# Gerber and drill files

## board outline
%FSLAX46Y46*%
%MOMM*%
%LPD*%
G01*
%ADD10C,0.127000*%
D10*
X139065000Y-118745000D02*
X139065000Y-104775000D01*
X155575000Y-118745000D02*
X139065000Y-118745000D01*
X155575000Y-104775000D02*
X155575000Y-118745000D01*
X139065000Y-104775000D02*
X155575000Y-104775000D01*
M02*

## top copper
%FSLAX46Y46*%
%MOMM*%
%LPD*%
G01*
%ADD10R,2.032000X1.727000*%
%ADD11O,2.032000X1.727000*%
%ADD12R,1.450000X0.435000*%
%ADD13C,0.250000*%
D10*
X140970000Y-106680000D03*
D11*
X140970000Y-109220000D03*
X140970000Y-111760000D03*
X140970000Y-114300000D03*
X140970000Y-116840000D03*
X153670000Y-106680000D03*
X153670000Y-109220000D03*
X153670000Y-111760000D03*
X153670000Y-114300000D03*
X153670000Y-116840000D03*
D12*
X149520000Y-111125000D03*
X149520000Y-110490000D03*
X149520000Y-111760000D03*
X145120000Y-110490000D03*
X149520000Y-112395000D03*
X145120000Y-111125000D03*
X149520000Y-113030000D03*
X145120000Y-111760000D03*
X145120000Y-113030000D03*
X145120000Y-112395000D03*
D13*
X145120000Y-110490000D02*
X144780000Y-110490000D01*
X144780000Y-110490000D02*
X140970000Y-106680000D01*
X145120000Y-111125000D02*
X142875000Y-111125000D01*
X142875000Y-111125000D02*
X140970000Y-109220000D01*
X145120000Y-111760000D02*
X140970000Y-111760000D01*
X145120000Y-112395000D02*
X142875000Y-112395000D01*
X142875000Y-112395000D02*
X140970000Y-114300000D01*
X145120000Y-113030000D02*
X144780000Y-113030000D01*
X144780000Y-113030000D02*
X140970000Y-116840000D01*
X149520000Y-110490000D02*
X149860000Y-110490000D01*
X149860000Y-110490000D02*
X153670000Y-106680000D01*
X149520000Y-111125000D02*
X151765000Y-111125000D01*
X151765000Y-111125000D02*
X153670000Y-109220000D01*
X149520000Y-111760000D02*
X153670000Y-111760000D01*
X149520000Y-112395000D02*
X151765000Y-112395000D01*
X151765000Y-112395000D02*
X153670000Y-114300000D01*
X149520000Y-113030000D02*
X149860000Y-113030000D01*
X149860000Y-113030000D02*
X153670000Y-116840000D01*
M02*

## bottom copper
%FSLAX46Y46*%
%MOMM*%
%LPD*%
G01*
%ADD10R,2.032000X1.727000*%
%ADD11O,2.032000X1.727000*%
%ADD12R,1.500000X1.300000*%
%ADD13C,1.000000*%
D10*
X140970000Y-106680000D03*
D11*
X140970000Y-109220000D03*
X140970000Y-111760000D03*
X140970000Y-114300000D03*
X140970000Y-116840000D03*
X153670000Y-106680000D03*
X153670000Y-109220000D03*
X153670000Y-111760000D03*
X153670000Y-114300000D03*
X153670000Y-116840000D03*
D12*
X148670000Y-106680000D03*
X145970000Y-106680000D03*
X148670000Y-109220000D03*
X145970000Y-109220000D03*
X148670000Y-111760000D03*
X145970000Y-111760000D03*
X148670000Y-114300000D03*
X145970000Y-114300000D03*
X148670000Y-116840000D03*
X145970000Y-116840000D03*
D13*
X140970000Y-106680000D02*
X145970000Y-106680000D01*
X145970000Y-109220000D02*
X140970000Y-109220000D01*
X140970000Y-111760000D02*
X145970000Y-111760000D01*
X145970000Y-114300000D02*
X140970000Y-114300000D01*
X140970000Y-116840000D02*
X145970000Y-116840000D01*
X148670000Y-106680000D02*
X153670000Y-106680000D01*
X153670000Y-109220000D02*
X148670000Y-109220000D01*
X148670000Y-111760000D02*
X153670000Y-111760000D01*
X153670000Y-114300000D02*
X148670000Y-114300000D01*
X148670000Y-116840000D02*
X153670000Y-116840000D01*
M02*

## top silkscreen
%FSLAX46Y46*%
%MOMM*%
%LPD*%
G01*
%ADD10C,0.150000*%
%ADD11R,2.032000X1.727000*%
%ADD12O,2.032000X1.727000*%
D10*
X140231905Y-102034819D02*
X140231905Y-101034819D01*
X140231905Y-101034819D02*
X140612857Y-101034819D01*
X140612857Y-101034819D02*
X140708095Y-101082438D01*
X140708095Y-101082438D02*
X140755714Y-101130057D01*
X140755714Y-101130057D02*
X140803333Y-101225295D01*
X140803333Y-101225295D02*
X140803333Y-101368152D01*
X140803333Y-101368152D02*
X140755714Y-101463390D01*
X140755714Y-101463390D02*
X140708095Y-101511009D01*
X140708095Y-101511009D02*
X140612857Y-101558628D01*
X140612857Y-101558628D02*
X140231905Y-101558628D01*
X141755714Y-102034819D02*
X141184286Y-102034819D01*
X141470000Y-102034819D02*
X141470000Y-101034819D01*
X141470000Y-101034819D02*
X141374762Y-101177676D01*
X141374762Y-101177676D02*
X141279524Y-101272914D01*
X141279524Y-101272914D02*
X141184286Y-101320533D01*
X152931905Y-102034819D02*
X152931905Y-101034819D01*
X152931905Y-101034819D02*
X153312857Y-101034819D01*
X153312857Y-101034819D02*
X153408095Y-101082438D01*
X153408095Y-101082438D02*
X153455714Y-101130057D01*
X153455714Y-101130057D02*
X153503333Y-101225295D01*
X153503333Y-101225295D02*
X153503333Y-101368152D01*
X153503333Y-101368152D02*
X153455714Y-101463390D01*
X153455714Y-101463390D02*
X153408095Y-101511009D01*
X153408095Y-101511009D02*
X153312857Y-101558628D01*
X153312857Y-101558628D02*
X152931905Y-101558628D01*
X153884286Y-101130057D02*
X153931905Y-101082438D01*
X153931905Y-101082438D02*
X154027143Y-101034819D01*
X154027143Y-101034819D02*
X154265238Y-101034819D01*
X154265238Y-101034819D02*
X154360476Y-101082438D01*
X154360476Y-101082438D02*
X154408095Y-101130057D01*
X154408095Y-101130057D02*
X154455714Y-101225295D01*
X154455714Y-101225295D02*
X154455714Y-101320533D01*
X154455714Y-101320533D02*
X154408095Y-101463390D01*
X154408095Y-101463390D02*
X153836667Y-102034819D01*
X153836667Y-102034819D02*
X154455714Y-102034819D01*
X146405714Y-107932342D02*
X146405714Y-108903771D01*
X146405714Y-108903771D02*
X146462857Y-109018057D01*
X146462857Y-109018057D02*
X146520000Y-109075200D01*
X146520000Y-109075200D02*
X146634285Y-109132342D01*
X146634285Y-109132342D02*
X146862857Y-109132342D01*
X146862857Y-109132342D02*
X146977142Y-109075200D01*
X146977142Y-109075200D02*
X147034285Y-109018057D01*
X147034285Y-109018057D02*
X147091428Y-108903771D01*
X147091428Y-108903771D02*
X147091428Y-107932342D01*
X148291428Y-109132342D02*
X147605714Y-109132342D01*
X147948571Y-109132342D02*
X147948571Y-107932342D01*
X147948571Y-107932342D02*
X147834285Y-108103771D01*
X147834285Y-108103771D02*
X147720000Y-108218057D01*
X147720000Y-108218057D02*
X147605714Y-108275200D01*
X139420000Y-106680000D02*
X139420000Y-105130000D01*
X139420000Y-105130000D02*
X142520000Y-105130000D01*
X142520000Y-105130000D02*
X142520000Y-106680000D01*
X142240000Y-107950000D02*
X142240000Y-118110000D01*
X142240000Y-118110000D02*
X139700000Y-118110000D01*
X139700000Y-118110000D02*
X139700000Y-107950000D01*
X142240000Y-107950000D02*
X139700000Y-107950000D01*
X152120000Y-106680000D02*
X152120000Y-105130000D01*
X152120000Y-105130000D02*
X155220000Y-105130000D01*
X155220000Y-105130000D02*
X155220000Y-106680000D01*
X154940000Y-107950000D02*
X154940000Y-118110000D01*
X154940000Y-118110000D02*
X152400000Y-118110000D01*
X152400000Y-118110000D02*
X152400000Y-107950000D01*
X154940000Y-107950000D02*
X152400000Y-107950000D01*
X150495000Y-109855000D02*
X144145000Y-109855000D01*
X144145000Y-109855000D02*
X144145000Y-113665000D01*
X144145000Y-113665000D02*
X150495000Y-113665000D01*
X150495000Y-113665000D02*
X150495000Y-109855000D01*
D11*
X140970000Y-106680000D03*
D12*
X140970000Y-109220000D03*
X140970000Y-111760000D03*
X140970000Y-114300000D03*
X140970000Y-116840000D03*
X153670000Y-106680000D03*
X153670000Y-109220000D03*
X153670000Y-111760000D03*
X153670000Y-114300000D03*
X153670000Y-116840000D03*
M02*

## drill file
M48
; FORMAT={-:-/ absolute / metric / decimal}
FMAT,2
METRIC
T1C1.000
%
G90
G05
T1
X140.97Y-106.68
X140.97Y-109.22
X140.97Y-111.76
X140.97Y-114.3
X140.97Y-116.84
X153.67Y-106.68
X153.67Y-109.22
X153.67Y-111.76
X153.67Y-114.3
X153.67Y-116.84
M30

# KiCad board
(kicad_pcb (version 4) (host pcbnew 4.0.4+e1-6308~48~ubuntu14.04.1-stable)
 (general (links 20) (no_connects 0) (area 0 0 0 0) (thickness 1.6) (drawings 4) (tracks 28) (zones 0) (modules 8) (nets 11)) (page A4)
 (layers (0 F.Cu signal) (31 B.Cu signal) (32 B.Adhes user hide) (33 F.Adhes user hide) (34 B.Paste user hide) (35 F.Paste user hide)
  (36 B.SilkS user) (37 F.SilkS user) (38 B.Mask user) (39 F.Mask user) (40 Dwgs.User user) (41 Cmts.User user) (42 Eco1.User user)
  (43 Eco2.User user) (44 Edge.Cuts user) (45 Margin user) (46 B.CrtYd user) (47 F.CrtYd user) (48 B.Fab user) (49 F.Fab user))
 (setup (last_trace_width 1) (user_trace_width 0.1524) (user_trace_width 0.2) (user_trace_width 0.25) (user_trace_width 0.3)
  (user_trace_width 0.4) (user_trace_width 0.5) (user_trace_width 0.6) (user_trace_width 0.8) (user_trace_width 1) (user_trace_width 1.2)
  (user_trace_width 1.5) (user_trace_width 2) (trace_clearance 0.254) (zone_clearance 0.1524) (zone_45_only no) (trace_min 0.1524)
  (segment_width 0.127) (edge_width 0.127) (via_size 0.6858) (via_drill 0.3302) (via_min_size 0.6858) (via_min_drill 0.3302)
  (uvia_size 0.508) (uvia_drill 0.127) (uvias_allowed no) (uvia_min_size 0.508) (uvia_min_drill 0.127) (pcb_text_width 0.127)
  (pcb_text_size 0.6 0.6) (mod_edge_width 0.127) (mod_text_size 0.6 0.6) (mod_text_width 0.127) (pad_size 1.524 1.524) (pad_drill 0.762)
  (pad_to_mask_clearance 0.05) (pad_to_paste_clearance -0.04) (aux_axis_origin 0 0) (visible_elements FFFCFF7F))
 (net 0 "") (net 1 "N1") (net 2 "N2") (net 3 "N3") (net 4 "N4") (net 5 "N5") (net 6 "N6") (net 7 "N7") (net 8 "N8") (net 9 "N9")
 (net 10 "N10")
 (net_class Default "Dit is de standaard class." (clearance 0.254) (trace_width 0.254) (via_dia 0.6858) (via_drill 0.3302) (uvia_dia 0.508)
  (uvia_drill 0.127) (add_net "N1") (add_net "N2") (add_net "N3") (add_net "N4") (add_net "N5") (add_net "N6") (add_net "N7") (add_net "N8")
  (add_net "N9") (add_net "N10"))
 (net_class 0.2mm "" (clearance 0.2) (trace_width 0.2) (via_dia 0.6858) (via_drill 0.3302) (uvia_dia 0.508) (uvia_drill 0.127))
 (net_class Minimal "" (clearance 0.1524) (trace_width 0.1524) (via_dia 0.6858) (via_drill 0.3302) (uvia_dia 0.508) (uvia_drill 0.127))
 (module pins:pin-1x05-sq (layer F.Cu) (at 140.97 106.68)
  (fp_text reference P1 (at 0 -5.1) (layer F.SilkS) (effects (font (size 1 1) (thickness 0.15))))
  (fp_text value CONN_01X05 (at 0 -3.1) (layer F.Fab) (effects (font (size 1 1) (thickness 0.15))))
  (fp_line (start -1.55 0) (end -1.55 -1.55) (layer F.SilkS) (width 0.15))
  (fp_line (start -1.55 -1.55) (end 1.55 -1.55) (layer F.SilkS) (width 0.15))
  (fp_line (start 1.55 -1.55) (end 1.55 0) (layer F.SilkS) (width 0.15))
  (fp_line (start 1.27 1.27) (end 1.27 11.43) (layer F.SilkS) (width 0.15))
  (fp_line (start 1.27 11.43) (end -1.27 11.43) (layer F.SilkS) (width 0.15))
  (fp_line (start -1.27 11.43) (end -1.27 1.27) (layer F.SilkS) (width 0.15))
  (fp_line (start 1.27 1.27) (end -1.27 1.27) (layer F.SilkS) (width 0.15))
  (pad 1 thru_hole rect (at 0 0) (size 2.032 1.727) (drill 1) (layers *.Cu *.Mask F.SilkS) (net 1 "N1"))
  (pad 2 thru_hole oval (at 0 2.54) (size 2.032 1.727) (drill 1) (layers *.Cu *.Mask F.SilkS) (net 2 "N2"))
  (pad 3 thru_hole oval (at 0 5.08) (size 2.032 1.727) (drill 1) (layers *.Cu *.Mask F.SilkS) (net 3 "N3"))
  (pad 4 thru_hole oval (at 0 7.62) (size 2.032 1.727) (drill 1) (layers *.Cu *.Mask F.SilkS) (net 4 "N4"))
  (pad 5 thru_hole oval (at 0 10.16) (size 2.032 1.727) (drill 1) (layers *.Cu *.Mask F.SilkS) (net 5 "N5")))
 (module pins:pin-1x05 (layer F.Cu) (at 153.67 106.68)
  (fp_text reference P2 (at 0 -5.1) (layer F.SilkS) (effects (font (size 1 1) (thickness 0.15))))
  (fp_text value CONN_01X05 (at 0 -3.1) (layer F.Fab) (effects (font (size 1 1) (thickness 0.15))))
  (fp_line (start -1.55 0) (end -1.55 -1.55) (layer F.SilkS) (width 0.15))
  (fp_line (start -1.55 -1.55) (end 1.55 -1.55) (layer F.SilkS) (width 0.15))
  (fp_line (start 1.55 -1.55) (end 1.55 0) (layer F.SilkS) (width 0.15))
  (fp_line (start 1.27 1.27) (end 1.27 11.43) (layer F.SilkS) (width 0.15))
  (fp_line (start 1.27 11.43) (end -1.27 11.43) (layer F.SilkS) (width 0.15))
  (fp_line (start -1.27 11.43) (end -1.27 1.27) (layer F.SilkS) (width 0.15))
  (fp_line (start 1.27 1.27) (end -1.27 1.27) (layer F.SilkS) (width 0.15))
  (pad 1 thru_hole oval (at 0 0) (size 2.032 1.727) (drill 1) (layers *.Cu *.Mask F.SilkS) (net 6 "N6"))
  (pad 2 thru_hole oval (at 0 2.54) (size 2.032 1.727) (drill 1) (layers *.Cu *.Mask F.SilkS) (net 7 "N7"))
  (pad 3 thru_hole oval (at 0 5.08) (size 2.032 1.727) (drill 1) (layers *.Cu *.Mask F.SilkS) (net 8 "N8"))
  (pad 4 thru_hole oval (at 0 7.62) (size 2.032 1.727) (drill 1) (layers *.Cu *.Mask F.SilkS) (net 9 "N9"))
  (pad 5 thru_hole oval (at 0 10.16) (size 2.032 1.727) (drill 1) (layers *.Cu *.Mask F.SilkS) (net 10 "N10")))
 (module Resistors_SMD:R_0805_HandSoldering (layer B.Cu) (at 147.32 106.68 180)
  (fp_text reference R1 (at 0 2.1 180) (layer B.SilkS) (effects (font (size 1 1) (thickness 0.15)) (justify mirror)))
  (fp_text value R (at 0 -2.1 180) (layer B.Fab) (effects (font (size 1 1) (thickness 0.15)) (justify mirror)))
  (pad 1 smd rect (at -1.35 0 180) (size 1.5 1.3) (layers B.Cu B.Paste B.Mask) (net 6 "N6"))
  (pad 2 smd rect (at 1.35 0 180) (size 1.5 1.3) (layers B.Cu B.Paste B.Mask) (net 1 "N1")))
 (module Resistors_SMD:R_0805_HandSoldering (layer B.Cu) (at 147.32 109.22 180)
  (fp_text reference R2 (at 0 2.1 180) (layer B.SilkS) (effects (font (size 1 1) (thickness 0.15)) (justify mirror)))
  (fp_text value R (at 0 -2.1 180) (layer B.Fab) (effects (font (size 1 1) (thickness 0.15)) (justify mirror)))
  (pad 1 smd rect (at -1.35 0 180) (size 1.5 1.3) (layers B.Cu B.Paste B.Mask) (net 7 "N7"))
  (pad 2 smd rect (at 1.35 0 180) (size 1.5 1.3) (layers B.Cu B.Paste B.Mask) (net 2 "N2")))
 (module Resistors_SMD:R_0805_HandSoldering (layer B.Cu) (at 147.32 111.76 180)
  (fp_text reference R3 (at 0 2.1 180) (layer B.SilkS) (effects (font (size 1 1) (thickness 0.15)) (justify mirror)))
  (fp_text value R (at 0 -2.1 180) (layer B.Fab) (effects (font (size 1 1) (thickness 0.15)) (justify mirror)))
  (pad 1 smd rect (at -1.35 0 180) (size 1.5 1.3) (layers B.Cu B.Paste B.Mask) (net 8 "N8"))
  (pad 2 smd rect (at 1.35 0 180) (size 1.5 1.3) (layers B.Cu B.Paste B.Mask) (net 3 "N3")))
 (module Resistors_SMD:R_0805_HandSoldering (layer B.Cu) (at 147.32 114.3 180)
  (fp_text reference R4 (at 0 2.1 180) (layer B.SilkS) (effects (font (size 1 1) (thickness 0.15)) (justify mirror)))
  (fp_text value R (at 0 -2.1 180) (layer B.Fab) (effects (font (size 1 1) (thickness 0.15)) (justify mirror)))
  (pad 1 smd rect (at -1.35 0 180) (size 1.5 1.3) (layers B.Cu B.Paste B.Mask) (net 9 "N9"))
  (pad 2 smd rect (at 1.35 0 180) (size 1.5 1.3) (layers B.Cu B.Paste B.Mask) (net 4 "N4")))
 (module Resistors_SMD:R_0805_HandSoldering (layer B.Cu) (at 147.32 116.84 180)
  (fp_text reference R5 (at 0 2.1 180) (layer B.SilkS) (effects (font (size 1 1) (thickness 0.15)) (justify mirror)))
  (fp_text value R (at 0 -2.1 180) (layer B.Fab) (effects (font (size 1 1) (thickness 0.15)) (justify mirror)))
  (pad 1 smd rect (at -1.35 0 180) (size 1.5 1.3) (layers B.Cu B.Paste B.Mask) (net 10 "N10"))
  (pad 2 smd rect (at 1.35 0 180) (size 1.5 1.3) (layers B.Cu B.Paste B.Mask) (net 5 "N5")))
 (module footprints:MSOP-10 (layer F.Cu) (at 147.32 111.76)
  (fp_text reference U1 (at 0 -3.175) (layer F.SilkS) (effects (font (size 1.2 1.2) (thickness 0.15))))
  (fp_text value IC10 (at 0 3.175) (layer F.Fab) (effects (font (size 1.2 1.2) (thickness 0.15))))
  (fp_line (start 3.175 -1.905) (end -3.175 -1.905) (layer F.SilkS) (width 0.15))
  (fp_line (start -3.175 -1.905) (end -3.175 1.905) (layer F.SilkS) (width 0.15))
  (fp_line (start -3.175 1.905) (end 3.175 1.905) (layer F.SilkS) (width 0.15))
  (fp_line (start 3.175 1.905) (end 3.175 -1.905) (layer F.SilkS) (width 0.15))
  (pad 9 smd rect (at 2.2 -0.635 270) (size 0.435 1.45) (layers F.Cu F.Paste F.Mask) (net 7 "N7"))
  (pad 10 smd rect (at 2.2 -1.27 270) (size 0.435 1.45) (layers F.Cu F.Paste F.Mask) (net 6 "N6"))
  (pad 8 smd rect (at 2.2 0 270) (size 0.435 1.45) (layers F.Cu F.Paste F.Mask) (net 8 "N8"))
  (pad 1 smd rect (at -2.2 -1.27 270) (size 0.435 1.45) (layers F.Cu F.Paste F.Mask) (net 1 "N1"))
  (pad 7 smd rect (at 2.2 0.635 270) (size 0.435 1.45) (layers F.Cu F.Paste F.Mask) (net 9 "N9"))
  (pad 2 smd rect (at -2.2 -0.635 270) (size 0.435 1.45) (layers F.Cu F.Paste F.Mask) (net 2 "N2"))
  (pad 6 smd rect (at 2.2 1.27 270) (size 0.435 1.45) (layers F.Cu F.Paste F.Mask) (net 10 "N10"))
  (pad 3 smd rect (at -2.2 0 270) (size 0.435 1.45) (layers F.Cu F.Paste F.Mask) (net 3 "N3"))
  (pad 5 smd rect (at -2.2 1.27 270) (size 0.435 1.45) (layers F.Cu F.Paste F.Mask) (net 5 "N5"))
  (pad 4 smd rect (at -2.2 0.635 270) (size 0.435 1.45) (layers F.Cu F.Paste F.Mask) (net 4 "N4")))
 (gr_line (start 139.065 118.745) (end 139.065 104.775) (angle 90) (layer Edge.Cuts) (width 0.127))
 (gr_line (start 155.575 118.745) (end 139.065 118.745) (angle 90) (layer Edge.Cuts) (width 0.127))
 (gr_line (start 155.575 104.775) (end 155.575 118.745) (angle 90) (layer Edge.Cuts) (width 0.127))
 (gr_line (start 139.065 104.775) (end 155.575 104.775) (angle 90) (layer Edge.Cuts) (width 0.127))
 (segment (start 140.97 106.68) (end 145.97 106.68) (width 1) (layer B.Cu) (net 1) (status C00000))
 (segment (start 145.12 110.49) (end 144.78 110.49) (width 0.25) (layer F.Cu) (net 1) (status C00000))
 (segment (start 144.78 110.49) (end 140.97 106.68) (width 0.25) (layer F.Cu) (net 1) (status C00000))
 (segment (start 145.97 109.22) (end 140.97 109.22) (width 1) (layer B.Cu) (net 2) (status C00000))
 (segment (start 145.12 111.125) (end 142.875 111.125) (width 0.25) (layer F.Cu) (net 2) (status 400000))
 (segment (start 142.875 111.125) (end 140.97 109.22) (width 0.25) (layer F.Cu) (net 2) (status 800000))
 (segment (start 140.97 111.76) (end 145.97 111.76) (width 1) (layer B.Cu) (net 3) (status C00000))
 (segment (start 145.12 111.76) (end 140.97 111.76) (width 0.25) (layer F.Cu) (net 3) (status C00000))
 (segment (start 145.97 114.3) (end 140.97 114.3) (width 1) (layer B.Cu) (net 4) (status C00000))
 (segment (start 145.12 112.395) (end 142.875 112.395) (width 0.25) (layer F.Cu) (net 4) (status 400000))
 (segment (start 142.875 112.395) (end 140.97 114.3) (width 0.25) (layer F.Cu) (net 4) (status 800000))
 (segment (start 140.97 116.84) (end 145.97 116.84) (width 1) (layer B.Cu) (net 5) (status C00000))
 (segment (start 145.12 113.03) (end 144.78 113.03) (width 0.25) (layer F.Cu) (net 5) (status C00000))
 (segment (start 144.78 113.03) (end 140.97 116.84) (width 0.25) (layer F.Cu) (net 5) (status C00000))
 (segment (start 148.67 106.68) (end 153.67 106.68) (width 1) (layer B.Cu) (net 6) (status C00000))
 (segment (start 149.52 110.49) (end 149.86 110.49) (width 0.25) (layer F.Cu) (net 6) (status C00000))
 (segment (start 149.86 110.49) (end 153.67 106.68) (width 0.25) (layer F.Cu) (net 6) (status C00000))
 (segment (start 153.67 109.22) (end 148.67 109.22) (width 1) (layer B.Cu) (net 7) (status C00000))
 (segment (start 149.52 111.125) (end 151.765 111.125) (width 0.25) (layer F.Cu) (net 7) (status 400000))
 (segment (start 151.765 111.125) (end 153.67 109.22) (width 0.25) (layer F.Cu) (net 7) (status 800000))
 (segment (start 148.67 111.76) (end 153.67 111.76) (width 1) (layer B.Cu) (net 8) (status C00000))
 (segment (start 149.52 111.76) (end 153.67 111.76) (width 0.25) (layer F.Cu) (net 8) (status C00000))
 (segment (start 153.67 114.3) (end 148.67 114.3) (width 1) (layer B.Cu) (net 9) (status C00000))
 (segment (start 149.52 112.395) (end 151.765 112.395) (width 0.25) (layer F.Cu) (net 9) (status 400000))
 (segment (start 151.765 112.395) (end 153.67 114.3) (width 0.25) (layer F.Cu) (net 9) (status 800000))
 (segment (start 148.67 116.84) (end 153.67 116.84) (width 1) (layer B.Cu) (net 10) (status C00000))
 (segment (start 149.52 113.03) (end 149.86 113.03) (width 0.25) (layer F.Cu) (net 10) (status C00000))
 (segment (start 149.86 113.03) (end 153.67 116.84) (width 0.25) (layer F.Cu) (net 10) (status C00000)))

